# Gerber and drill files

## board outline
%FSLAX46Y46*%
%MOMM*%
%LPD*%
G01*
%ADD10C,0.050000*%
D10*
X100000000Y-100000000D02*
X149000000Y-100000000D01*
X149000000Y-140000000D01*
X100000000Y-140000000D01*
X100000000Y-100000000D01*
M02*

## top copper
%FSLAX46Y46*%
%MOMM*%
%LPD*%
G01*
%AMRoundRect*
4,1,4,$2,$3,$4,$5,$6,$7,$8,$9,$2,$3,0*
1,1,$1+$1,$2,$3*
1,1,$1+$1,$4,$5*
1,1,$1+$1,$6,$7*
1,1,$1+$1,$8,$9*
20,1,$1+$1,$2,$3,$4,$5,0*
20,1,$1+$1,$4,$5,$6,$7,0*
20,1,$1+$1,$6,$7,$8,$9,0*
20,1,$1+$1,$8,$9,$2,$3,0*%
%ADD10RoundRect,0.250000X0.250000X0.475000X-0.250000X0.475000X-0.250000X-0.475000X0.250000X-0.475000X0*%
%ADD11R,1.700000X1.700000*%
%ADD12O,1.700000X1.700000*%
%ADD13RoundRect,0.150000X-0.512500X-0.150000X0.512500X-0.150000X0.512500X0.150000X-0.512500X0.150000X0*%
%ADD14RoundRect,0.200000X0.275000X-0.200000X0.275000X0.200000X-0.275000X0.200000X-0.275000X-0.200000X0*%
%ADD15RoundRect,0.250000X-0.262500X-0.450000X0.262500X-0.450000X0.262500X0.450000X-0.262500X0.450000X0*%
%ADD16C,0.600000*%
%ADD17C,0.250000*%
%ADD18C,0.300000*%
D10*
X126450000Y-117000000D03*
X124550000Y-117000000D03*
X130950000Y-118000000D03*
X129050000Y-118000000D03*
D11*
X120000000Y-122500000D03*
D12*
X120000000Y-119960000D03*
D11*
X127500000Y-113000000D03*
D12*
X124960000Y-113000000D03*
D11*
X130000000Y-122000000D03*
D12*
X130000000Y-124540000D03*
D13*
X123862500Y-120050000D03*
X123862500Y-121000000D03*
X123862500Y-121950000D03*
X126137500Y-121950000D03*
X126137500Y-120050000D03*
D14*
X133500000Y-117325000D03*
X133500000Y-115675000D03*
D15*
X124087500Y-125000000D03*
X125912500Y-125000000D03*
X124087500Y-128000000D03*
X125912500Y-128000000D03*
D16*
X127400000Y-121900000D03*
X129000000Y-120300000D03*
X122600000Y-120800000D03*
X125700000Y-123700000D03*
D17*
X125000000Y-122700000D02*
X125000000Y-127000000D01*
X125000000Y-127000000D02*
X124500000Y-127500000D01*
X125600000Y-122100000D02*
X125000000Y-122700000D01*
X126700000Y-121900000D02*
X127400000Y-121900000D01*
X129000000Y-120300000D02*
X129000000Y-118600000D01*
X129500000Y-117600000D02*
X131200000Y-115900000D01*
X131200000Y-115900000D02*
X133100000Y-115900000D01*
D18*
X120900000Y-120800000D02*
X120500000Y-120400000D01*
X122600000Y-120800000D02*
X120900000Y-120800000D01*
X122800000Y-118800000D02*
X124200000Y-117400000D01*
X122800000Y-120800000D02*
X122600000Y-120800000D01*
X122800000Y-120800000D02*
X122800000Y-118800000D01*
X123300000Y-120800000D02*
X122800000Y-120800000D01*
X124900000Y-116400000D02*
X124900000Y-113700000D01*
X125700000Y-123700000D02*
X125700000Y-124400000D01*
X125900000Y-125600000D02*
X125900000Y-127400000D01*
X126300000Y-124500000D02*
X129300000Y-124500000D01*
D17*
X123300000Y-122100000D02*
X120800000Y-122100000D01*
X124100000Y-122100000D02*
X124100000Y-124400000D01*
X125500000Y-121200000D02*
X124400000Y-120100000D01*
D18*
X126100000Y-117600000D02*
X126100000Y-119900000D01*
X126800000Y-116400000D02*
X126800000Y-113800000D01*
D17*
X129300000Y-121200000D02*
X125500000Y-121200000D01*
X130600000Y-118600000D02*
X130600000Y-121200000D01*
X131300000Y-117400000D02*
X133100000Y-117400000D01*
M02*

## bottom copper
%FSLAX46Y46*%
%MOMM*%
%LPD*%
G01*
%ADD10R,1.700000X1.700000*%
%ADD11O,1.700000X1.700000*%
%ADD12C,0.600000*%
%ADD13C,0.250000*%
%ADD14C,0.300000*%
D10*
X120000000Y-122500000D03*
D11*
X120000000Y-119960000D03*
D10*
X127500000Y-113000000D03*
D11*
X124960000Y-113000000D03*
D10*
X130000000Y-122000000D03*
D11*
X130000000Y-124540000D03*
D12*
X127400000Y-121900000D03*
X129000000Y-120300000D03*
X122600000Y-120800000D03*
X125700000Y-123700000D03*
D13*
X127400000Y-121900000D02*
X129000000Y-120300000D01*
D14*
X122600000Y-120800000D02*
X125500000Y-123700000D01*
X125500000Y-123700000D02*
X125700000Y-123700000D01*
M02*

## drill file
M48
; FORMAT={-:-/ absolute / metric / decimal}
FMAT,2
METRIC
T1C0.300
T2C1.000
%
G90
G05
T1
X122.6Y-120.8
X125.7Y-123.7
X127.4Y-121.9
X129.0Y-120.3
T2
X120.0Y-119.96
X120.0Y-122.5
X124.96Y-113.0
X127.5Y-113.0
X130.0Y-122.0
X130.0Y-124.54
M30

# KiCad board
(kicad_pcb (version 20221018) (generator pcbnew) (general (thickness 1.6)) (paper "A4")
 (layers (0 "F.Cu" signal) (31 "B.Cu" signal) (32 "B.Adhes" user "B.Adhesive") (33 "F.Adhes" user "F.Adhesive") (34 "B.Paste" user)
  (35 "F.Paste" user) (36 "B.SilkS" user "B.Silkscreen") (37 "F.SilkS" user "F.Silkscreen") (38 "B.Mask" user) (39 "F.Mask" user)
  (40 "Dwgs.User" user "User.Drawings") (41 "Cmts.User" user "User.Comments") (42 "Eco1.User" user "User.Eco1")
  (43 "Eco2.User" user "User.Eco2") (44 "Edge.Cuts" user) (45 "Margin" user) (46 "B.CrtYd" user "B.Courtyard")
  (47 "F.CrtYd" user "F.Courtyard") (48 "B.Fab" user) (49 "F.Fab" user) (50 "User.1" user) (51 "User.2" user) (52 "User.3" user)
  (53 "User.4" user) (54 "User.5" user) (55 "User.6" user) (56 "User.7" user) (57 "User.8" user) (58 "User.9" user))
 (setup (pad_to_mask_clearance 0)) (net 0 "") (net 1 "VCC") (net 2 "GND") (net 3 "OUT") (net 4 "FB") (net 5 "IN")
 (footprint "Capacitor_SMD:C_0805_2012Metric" (layer "F.Cu") (at 125.5 117 180)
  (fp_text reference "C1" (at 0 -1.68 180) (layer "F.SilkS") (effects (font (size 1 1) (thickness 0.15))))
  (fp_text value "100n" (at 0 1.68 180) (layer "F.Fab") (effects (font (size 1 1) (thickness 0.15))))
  (pad "1" smd roundrect (at -0.95 0 180) (size 1 1.45) (layers "F.Cu" "F.Paste" "F.Mask") (roundrect_rratio 0.25) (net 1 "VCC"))
  (pad "2" smd roundrect (at 0.95 0 180) (size 1 1.45) (layers "F.Cu" "F.Paste" "F.Mask") (roundrect_rratio 0.25) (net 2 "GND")))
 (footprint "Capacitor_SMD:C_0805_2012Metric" (layer "F.Cu") (at 130 118 180)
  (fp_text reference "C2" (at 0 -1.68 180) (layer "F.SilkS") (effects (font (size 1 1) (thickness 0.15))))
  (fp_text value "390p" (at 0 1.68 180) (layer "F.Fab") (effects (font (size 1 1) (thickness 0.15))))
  (pad "1" smd roundrect (at -0.95 0 180) (size 1 1.45) (layers "F.Cu" "F.Paste" "F.Mask") (roundrect_rratio 0.25) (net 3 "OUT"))
  (pad "2" smd roundrect (at 0.95 0 180) (size 1 1.45) (layers "F.Cu" "F.Paste" "F.Mask") (roundrect_rratio 0.25) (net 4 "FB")))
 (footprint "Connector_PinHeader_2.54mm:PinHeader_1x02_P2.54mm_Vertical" (layer "F.Cu") (at 120 122.5 180)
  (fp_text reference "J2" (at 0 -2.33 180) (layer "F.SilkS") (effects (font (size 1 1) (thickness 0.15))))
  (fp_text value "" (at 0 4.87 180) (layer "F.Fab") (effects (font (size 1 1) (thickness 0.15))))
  (pad "1" thru_hole rect (at 0 0 180) (size 1.7 1.7) (drill 1) (layers "*.Cu" "*.Mask") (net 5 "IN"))
  (pad "2" thru_hole oval (at 0 2.54 180) (size 1.7 1.7) (drill 1) (layers "*.Cu" "*.Mask") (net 2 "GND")))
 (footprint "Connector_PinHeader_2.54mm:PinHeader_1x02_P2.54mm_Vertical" (layer "F.Cu") (at 127.5 113 -90)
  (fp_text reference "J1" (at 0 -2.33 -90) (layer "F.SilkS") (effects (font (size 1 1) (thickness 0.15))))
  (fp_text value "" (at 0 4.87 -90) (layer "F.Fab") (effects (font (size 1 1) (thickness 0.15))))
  (pad "1" thru_hole rect (at 0 0 270) (size 1.7 1.7) (drill 1) (layers "*.Cu" "*.Mask") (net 1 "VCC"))
  (pad "2" thru_hole oval (at 0 2.54 270) (size 1.7 1.7) (drill 1) (layers "*.Cu" "*.Mask") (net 2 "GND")))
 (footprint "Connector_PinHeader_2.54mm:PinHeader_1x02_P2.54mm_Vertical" (layer "F.Cu") (at 130 122)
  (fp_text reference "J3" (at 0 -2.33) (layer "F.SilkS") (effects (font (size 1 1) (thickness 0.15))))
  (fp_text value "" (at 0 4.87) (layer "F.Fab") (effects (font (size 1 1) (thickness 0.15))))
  (pad "1" thru_hole rect (at 0 0) (size 1.7 1.7) (drill 1) (layers "*.Cu" "*.Mask") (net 3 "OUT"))
  (pad "2" thru_hole oval (at 0 2.54) (size 1.7 1.7) (drill 1) (layers "*.Cu" "*.Mask") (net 2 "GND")))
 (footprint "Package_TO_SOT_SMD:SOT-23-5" (layer "F.Cu") (at 125 121)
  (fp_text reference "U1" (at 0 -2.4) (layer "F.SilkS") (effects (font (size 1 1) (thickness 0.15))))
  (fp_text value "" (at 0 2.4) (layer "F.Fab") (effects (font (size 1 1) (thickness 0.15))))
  (pad "1" smd roundrect (at -1.1375 -0.95) (size 1.325 0.6) (layers "F.Cu" "F.Paste" "F.Mask") (roundrect_rratio 0.25) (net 3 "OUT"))
  (pad "2" smd roundrect (at -1.1375 0) (size 1.325 0.6) (layers "F.Cu" "F.Paste" "F.Mask") (roundrect_rratio 0.25) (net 2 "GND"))
  (pad "3" smd roundrect (at -1.1375 0.95) (size 1.325 0.6) (layers "F.Cu" "F.Paste" "F.Mask") (roundrect_rratio 0.25) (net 5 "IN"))
  (pad "4" smd roundrect (at 1.1375 0.95) (size 1.325 0.6) (layers "F.Cu" "F.Paste" "F.Mask") (roundrect_rratio 0.25) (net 4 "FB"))
  (pad "5" smd roundrect (at 1.1375 -0.95) (size 1.325 0.6) (layers "F.Cu" "F.Paste" "F.Mask") (roundrect_rratio 0.25) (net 1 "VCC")))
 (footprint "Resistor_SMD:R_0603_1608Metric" (layer "F.Cu") (at 133.5 116.5 90)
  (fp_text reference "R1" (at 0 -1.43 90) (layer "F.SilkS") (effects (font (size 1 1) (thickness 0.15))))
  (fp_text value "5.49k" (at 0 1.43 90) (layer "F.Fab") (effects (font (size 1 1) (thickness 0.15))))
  (pad "1" smd roundrect (at -0.825 0 90) (size 0.8 0.95) (layers "F.Cu" "F.Paste" "F.Mask") (roundrect_rratio 0.25) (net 3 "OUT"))
  (pad "2" smd roundrect (at 0.825 0 90) (size 0.8 0.95) (layers "F.Cu" "F.Paste" "F.Mask") (roundrect_rratio 0.25) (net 4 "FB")))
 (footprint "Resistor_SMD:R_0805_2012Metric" (layer "F.Cu") (at 125 125)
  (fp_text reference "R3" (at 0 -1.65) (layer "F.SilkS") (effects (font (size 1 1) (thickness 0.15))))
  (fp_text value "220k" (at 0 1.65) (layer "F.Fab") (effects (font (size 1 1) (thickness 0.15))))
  (pad "1" smd roundrect (at -0.9125 0) (size 1.025 1.4) (layers "F.Cu" "F.Paste" "F.Mask") (roundrect_rratio 0.243902) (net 5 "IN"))
  (pad "2" smd roundrect (at 0.9125 0) (size 1.025 1.4) (layers "F.Cu" "F.Paste" "F.Mask") (roundrect_rratio 0.243902) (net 2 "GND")))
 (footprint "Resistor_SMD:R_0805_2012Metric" (layer "F.Cu") (at 125 128)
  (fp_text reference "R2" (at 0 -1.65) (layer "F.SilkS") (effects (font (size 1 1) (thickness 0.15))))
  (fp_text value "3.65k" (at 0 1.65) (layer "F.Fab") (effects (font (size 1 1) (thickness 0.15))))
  (pad "1" smd roundrect (at -0.9125 0) (size 1.025 1.4) (layers "F.Cu" "F.Paste" "F.Mask") (roundrect_rratio 0.243902) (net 4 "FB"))
  (pad "2" smd roundrect (at 0.9125 0) (size 1.025 1.4) (layers "F.Cu" "F.Paste" "F.Mask") (roundrect_rratio 0.243902) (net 2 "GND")))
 (gr_rect (start 100 100) (end 149 140) (stroke (width 0.05) (type default)) (fill none) (layer "Edge.Cuts"))
 (segment (start 125 122.7) (end 125 127) (width 0.25) (layer "F.Cu") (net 4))
 (segment (start 125 127) (end 124.5 127.5) (width 0.25) (layer "F.Cu") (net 4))
 (segment (start 125.6 122.1) (end 125 122.7) (width 0.25) (layer "F.Cu") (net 4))
 (segment (start 126.7 121.9) (end 127.4 121.9) (width 0.25) (layer "F.Cu") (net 4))
 (segment (start 129 120.3) (end 129 118.6) (width 0.25) (layer "F.Cu") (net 4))
 (segment (start 129.5 117.6) (end 131.2 115.9) (width 0.25) (layer "F.Cu") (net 4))
 (segment (start 131.2 115.9) (end 133.1 115.9) (width 0.25) (layer "F.Cu") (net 4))
 (via (at 127.4 121.9) (size 0.6) (drill 0.3) (layers "F.Cu" "B.Cu") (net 4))
 (via (at 129 120.3) (size 0.6) (drill 0.3) (layers "F.Cu" "B.Cu") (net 4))
 (segment (start 120.9 120.8) (end 120.5 120.4) (width 0.3) (layer "F.Cu") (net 2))
 (segment (start 122.6 120.8) (end 120.9 120.8) (width 0.3) (layer "F.Cu") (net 2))
 (segment (start 122.8 118.8) (end 124.2 117.4) (width 0.3) (layer "F.Cu") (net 2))
 (segment (start 122.8 120.8) (end 122.6 120.8) (width 0.3) (layer "F.Cu") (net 2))
 (segment (start 122.8 120.8) (end 122.8 118.8) (width 0.3) (layer "F.Cu") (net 2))
 (segment (start 123.3 120.8) (end 122.8 120.8) (width 0.3) (layer "F.Cu") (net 2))
 (segment (start 124.9 116.4) (end 124.9 113.7) (width 0.3) (layer "F.Cu") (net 2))
 (segment (start 125.7 123.7) (end 125.7 124.4) (width 0.3) (layer "F.Cu") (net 2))
 (segment (start 125.9 125.6) (end 125.9 127.4) (width 0.3) (layer "F.Cu") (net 2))
 (segment (start 126.3 124.5) (end 129.3 124.5) (width 0.3) (layer "F.Cu") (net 2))
 (segment (start 127.4 121.9) (end 129 120.3) (width 0.25) (layer "B.Cu") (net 4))
 (via (at 122.6 120.8) (size 0.6) (drill 0.3) (layers "F.Cu" "B.Cu") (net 2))
 (via (at 125.7 123.7) (size 0.6) (drill 0.3) (layers "F.Cu" "B.Cu") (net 2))
 (segment (start 122.6 120.8) (end 125.5 123.7) (width 0.3) (layer "B.Cu") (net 2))
 (segment (start 123.3 122.1) (end 120.8 122.1) (width 0.25) (layer "F.Cu") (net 5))
 (segment (start 124.1 122.1) (end 124.1 124.4) (width 0.25) (layer "F.Cu") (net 5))
 (segment (start 125.5 121.2) (end 124.4 120.1) (width 0.25) (layer "F.Cu") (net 3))
 (segment (start 125.5 123.7) (end 125.7 123.7) (width 0.3) (layer "B.Cu") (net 2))
 (segment (start 126.1 117.6) (end 126.1 119.9) (width 0.3) (layer "F.Cu") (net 1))
 (segment (start 126.8 116.4) (end 126.8 113.8) (width 0.3) (layer "F.Cu") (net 1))
 (segment (start 129.3 121.2) (end 125.5 121.2) (width 0.25) (layer "F.Cu") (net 3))
 (segment (start 130.6 118.6) (end 130.6 121.2) (width 0.25) (layer "F.Cu") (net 3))
 (segment (start 131.3 117.4) (end 133.1 117.4) (width 0.25) (layer "F.Cu") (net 3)))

